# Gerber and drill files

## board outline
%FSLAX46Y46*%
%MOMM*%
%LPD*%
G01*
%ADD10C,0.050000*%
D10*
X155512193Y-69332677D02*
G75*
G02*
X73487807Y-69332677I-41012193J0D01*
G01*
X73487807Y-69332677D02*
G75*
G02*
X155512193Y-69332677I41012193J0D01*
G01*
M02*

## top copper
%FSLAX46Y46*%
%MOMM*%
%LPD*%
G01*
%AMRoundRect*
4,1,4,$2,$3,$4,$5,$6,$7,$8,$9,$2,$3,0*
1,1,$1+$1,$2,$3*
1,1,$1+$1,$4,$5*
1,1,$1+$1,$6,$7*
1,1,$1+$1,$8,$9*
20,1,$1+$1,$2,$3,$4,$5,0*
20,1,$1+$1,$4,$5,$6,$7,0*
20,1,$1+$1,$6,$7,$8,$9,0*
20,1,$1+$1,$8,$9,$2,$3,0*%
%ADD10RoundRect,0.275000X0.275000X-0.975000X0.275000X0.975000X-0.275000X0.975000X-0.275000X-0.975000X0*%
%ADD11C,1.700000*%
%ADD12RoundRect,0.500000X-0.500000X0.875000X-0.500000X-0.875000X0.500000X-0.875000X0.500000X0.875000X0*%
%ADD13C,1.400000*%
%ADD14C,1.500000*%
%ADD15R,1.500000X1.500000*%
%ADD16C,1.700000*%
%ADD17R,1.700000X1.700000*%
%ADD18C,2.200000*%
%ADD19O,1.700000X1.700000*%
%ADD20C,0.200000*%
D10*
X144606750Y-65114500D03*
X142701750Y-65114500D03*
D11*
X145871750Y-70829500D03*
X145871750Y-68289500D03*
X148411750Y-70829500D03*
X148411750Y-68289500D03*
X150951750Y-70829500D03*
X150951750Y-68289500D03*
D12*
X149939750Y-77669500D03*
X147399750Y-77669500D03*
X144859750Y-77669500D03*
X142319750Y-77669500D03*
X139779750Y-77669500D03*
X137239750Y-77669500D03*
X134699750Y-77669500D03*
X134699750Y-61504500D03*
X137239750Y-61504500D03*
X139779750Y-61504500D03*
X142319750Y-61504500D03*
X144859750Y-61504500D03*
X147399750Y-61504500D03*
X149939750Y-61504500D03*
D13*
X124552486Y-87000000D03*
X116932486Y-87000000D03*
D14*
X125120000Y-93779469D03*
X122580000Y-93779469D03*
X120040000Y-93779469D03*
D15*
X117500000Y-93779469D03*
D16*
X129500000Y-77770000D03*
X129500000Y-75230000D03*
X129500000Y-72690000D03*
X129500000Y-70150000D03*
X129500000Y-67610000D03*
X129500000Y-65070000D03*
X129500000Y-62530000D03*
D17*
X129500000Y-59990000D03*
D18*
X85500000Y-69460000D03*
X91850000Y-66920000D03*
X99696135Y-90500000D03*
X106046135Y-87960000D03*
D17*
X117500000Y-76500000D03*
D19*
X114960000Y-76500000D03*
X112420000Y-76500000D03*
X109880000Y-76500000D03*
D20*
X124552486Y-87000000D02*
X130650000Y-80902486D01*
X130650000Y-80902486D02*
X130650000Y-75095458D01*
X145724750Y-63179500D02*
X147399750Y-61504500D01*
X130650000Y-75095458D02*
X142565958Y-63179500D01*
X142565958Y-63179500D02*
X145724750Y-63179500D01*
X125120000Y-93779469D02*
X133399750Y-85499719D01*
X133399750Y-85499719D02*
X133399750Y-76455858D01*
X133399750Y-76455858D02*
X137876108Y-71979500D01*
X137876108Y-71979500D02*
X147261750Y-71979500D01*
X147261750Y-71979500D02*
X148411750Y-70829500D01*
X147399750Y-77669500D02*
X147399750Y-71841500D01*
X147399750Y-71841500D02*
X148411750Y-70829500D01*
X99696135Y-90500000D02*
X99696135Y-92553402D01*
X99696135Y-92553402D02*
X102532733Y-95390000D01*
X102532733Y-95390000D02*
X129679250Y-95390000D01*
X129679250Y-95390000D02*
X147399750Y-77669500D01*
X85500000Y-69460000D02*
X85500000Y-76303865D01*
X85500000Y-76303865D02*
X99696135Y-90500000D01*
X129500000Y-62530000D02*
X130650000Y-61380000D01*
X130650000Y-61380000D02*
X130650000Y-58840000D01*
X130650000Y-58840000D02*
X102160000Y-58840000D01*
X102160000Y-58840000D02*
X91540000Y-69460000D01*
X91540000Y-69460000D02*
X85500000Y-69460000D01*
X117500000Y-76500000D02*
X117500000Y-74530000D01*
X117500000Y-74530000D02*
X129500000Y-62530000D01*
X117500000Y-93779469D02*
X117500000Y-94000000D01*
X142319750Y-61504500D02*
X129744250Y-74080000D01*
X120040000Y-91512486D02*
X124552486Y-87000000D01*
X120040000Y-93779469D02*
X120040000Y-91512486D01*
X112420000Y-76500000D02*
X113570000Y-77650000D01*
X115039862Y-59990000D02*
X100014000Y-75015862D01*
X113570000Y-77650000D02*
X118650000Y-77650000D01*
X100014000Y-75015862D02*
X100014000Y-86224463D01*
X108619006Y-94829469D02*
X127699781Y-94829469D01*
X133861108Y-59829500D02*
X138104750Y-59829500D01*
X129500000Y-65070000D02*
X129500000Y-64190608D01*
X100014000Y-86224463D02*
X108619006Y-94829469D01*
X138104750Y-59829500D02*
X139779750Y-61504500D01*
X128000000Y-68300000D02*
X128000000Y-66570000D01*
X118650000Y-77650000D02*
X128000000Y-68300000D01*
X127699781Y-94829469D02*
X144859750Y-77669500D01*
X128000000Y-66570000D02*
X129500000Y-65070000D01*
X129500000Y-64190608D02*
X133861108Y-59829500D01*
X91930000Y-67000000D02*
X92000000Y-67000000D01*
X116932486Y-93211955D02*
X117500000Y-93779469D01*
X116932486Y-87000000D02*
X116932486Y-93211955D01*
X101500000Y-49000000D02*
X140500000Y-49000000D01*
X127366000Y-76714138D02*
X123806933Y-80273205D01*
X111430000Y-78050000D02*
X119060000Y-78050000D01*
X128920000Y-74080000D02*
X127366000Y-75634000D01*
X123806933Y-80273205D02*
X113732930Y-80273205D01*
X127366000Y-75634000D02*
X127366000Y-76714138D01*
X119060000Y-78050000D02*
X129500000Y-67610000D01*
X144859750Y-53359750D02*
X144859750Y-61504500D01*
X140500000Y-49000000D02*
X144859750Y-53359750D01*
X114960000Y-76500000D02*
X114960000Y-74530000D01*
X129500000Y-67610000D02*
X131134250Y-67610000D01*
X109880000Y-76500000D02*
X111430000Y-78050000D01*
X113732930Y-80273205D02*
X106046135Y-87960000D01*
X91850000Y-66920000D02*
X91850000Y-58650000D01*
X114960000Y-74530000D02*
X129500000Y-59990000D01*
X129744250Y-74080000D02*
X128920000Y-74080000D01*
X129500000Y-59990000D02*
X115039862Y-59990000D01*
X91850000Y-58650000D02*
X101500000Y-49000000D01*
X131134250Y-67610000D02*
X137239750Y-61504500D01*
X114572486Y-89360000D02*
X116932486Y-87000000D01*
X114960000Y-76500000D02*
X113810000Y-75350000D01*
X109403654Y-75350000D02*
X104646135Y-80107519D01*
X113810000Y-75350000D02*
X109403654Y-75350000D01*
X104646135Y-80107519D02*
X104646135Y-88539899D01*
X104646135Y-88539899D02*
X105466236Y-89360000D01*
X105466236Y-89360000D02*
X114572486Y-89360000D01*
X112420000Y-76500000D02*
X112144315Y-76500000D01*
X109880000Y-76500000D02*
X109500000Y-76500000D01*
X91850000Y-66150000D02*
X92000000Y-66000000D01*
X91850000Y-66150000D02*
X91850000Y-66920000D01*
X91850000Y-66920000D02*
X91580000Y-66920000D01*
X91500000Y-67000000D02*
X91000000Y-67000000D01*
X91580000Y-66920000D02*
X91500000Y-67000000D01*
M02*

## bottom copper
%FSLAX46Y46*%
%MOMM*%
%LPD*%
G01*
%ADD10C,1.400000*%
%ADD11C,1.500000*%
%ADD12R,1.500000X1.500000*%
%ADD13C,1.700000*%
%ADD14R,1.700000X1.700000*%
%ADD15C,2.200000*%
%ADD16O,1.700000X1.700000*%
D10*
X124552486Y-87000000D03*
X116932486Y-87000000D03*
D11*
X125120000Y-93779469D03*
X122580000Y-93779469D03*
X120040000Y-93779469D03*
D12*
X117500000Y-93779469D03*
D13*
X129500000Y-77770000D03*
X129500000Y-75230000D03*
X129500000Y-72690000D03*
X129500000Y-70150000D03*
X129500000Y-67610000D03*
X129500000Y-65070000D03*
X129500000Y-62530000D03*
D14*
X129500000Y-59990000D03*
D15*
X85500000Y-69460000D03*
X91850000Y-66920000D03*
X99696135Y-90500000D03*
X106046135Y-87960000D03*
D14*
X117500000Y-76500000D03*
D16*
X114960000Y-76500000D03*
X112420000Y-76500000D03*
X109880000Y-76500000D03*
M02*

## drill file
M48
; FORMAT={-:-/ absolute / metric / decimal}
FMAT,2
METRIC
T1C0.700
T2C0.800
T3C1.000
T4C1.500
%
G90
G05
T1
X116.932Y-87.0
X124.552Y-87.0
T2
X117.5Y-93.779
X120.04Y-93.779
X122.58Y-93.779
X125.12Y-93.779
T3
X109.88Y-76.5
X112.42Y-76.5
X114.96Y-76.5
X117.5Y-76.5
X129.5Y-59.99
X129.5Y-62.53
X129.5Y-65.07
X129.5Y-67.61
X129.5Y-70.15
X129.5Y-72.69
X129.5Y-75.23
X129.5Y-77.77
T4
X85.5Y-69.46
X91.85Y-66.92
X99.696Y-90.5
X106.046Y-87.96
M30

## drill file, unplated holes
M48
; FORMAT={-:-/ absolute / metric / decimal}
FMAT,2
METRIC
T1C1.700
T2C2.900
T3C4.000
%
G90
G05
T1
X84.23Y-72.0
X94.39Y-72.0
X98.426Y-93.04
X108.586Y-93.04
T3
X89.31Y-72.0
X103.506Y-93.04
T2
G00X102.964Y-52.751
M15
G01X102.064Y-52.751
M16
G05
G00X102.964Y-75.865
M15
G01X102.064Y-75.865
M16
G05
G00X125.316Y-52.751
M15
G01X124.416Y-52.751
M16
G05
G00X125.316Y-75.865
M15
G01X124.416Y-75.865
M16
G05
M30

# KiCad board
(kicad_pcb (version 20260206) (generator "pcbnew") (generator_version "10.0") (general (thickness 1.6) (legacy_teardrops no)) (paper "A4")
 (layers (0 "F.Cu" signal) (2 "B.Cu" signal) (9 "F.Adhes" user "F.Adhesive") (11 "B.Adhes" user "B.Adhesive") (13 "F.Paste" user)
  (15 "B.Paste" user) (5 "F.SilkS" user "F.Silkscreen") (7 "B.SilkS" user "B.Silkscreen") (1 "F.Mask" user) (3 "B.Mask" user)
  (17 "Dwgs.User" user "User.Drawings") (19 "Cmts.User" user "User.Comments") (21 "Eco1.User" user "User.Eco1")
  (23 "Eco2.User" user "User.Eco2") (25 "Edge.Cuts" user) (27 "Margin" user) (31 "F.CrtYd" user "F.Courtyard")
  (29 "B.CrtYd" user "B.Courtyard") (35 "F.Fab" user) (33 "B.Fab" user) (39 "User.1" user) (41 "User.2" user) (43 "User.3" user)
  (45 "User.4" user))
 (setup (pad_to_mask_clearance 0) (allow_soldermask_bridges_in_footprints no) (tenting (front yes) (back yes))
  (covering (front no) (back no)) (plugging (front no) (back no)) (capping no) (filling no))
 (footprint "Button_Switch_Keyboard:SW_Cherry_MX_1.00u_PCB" (layer "F.Cu") (at 106.046135 87.96)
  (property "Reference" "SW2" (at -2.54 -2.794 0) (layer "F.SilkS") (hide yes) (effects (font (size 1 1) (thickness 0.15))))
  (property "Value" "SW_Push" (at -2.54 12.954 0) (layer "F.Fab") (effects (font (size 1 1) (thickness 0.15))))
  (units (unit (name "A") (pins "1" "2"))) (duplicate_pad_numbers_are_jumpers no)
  (pad "" np_thru_hole circle (at -7.62 5.08) (size 1.7 1.7) (drill 1.7) (layers "*.Cu" "*.Mask"))
  (pad "" np_thru_hole circle (at -2.54 5.08) (size 4 4) (drill 4) (layers "*.Cu" "*.Mask"))
  (pad "" np_thru_hole circle (at 2.54 5.08) (size 1.7 1.7) (drill 1.7) (layers "*.Cu" "*.Mask"))
  (pad "1" thru_hole circle (at 0 0) (size 2.2 2.2) (drill 1.5) (layers "*.Cu" "*.Mask") (remove_unused_layers no) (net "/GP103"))
  (pad "2" thru_hole circle (at -6.35 2.54) (size 2.2 2.2) (drill 1.5) (layers "*.Cu" "*.Mask") (remove_unused_layers no) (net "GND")))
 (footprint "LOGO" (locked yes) (layer "F.Cu") (at 114.5 69.332677)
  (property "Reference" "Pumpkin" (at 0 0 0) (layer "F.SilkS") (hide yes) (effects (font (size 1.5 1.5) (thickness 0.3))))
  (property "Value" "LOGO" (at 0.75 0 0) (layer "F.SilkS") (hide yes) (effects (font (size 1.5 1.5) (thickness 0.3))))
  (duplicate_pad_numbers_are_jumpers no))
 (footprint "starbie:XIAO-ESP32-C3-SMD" (layer "F.Cu") (at 131.81975 60.6695 -90)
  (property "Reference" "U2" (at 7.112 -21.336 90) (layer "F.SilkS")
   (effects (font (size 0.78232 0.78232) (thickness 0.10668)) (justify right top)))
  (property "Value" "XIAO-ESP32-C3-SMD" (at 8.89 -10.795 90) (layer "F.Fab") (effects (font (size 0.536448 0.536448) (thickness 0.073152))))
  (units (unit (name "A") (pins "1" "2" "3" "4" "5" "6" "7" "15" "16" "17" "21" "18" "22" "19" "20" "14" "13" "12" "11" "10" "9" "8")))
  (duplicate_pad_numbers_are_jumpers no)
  (pad "1" smd roundrect (at 0.835 -18.12 270) (size 2.75 2) (layers "F.Cu" "F.Mask" "F.Paste") (roundrect_rratio 0.25)
   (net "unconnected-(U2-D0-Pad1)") (solder_mask_margin 0.0508) (thermal_bridge_angle 45))
  (pad "2" smd roundrect (at 0.835 -15.58 270) (size 2.75 2) (layers "F.Cu" "F.Mask" "F.Paste") (roundrect_rratio 0.25) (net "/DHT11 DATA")
   (solder_mask_margin 0.0508) (thermal_bridge_angle 45))
  (pad "3" smd roundrect (at 0.835 -13.04 270) (size 2.75 2) (layers "F.Cu" "F.Mask" "F.Paste") (roundrect_rratio 0.25) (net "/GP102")
   (solder_mask_margin 0.0508) (thermal_bridge_angle 45))
  (pad "4" smd roundrect (at 0.835 -10.5 270) (size 2.75 2) (layers "F.Cu" "F.Mask" "F.Paste") (roundrect_rratio 0.25) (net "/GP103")
   (solder_mask_margin 0.0508) (thermal_bridge_angle 45))
  (pad "5" smd roundrect (at 0.835 -7.96 270) (size 2.75 2) (layers "F.Cu" "F.Mask" "F.Paste") (roundrect_rratio 0.25) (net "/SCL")
   (solder_mask_margin 0.0508) (thermal_bridge_angle 45))
  (pad "6" smd roundrect (at 0.835 -5.42 270) (size 2.75 2) (layers "F.Cu" "F.Mask" "F.Paste") (roundrect_rratio 0.25) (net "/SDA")
   (solder_mask_margin 0.0508) (thermal_bridge_angle 45))
  (pad "7" smd roundrect (at 0.835 -2.88 270) (size 2.75 2) (layers "F.Cu" "F.Mask" "F.Paste") (roundrect_rratio 0.25)
   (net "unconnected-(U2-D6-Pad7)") (solder_mask_margin 0.0508) (thermal_bridge_angle 45))
  (pad "8" smd roundrect (at 17 -2.88 270) (size 2.75 2) (layers "F.Cu" "F.Mask" "F.Paste") (roundrect_rratio 0.25)
   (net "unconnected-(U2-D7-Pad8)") (solder_mask_margin 0.0508) (thermal_bridge_angle 45))
  (pad "9" smd roundrect (at 17 -5.42 270) (size 2.75 2) (layers "F.Cu" "F.Mask" "F.Paste") (roundrect_rratio 0.25)
   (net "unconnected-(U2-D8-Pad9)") (solder_mask_margin 0.0508) (thermal_bridge_angle 45))
  (pad "10" smd roundrect (at 17 -7.96 270) (size 2.75 2) (layers "F.Cu" "F.Mask" "F.Paste") (roundrect_rratio 0.25)
   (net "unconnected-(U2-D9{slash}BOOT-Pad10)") (solder_mask_margin 0.0508) (thermal_bridge_angle 45))
  (pad "11" smd roundrect (at 17 -10.5 270) (size 2.75 2) (layers "F.Cu" "F.Mask" "F.Paste") (roundrect_rratio 0.25)
   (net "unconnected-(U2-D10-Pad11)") (solder_mask_margin 0.0508) (thermal_bridge_angle 45))
  (pad "12" smd roundrect (at 17 -13.04 270) (size 2.75 2) (layers "F.Cu" "F.Mask" "F.Paste") (roundrect_rratio 0.25) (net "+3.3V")
   (solder_mask_margin 0.0508) (thermal_bridge_angle 45))
  (pad "13" smd roundrect (at 17 -15.58 270) (size 2.75 2) (layers "F.Cu" "F.Mask" "F.Paste") (roundrect_rratio 0.25) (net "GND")
   (solder_mask_margin 0.0508) (thermal_bridge_angle 45))
  (pad "14" smd roundrect (at 17 -18.12 270) (size 2.75 2) (layers "F.Cu" "F.Mask" "F.Paste") (roundrect_rratio 0.25) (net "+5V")
   (solder_mask_margin 0.0508) (thermal_bridge_angle 45))
  (pad "15" smd circle (at 7.62 -19.132 270) (size 1.7 1.7) (layers "F.Cu" "F.Mask" "F.Paste") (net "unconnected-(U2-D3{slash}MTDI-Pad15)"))
  (pad "16" smd circle (at 10.16 -19.132 270) (size 1.7 1.7) (layers "F.Cu" "F.Mask" "F.Paste") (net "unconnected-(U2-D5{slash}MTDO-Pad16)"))
  (pad "17" smd circle (at 7.62 -16.592 270) (size 1.7 1.7) (layers "F.Cu" "F.Mask" "F.Paste") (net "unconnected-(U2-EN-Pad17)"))
  (pad "18" smd circle (at 10.16 -16.592 270) (size 1.7 1.7) (layers "F.Cu" "F.Mask" "F.Paste") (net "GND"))
  (pad "19" smd circle (at 7.62 -14.052 270) (size 1.7 1.7) (layers "F.Cu" "F.Mask" "F.Paste") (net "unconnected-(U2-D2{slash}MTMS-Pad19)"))
  (pad "20" smd circle (at 10.16 -14.052 270) (size 1.7 1.7) (layers "F.Cu" "F.Mask" "F.Paste") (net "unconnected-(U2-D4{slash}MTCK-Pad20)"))
  (pad "21" smd roundrect (at 4.445 -10.882 90) (size 2.5 1.1) (layers "F.Cu" "F.Mask" "F.Paste") (roundrect_rratio 0.25)
   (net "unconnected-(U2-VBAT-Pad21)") (thermal_bridge_angle 45))
  (pad "22" smd roundrect (at 4.445 -12.787 90) (size 2.5 1.1) (layers "F.Cu" "F.Mask" "F.Paste") (roundrect_rratio 0.25)
   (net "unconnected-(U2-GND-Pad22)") (thermal_bridge_angle 45)))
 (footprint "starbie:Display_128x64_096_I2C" (layer "F.Cu") (at 113.69 76.5 180)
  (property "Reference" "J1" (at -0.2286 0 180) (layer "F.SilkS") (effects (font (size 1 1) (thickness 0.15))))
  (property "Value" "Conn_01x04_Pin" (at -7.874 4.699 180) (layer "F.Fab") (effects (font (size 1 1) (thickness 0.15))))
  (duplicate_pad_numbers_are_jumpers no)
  (pad "" np_thru_hole oval (at -11.176 0.635 180) (size 3.8 2.9) (drill oval 3.8 2.9) (layers "*.Cu" "*.Mask"))
  (pad "" np_thru_hole oval (at -11.176 23.749 180) (size 3.8 2.9) (drill oval 3.8 2.9) (layers "*.Cu" "*.Mask"))
  (pad "" np_thru_hole oval (at 11.176 0.635 180) (size 3.8 2.9) (drill oval 3.8 2.9) (layers "*.Cu" "*.Mask"))
  (pad "" np_thru_hole oval (at 11.176 23.749 180) (size 3.8 2.9) (drill oval 3.8 2.9) (layers "*.Cu" "*.Mask"))
  (pad "1" thru_hole rect (at -3.81 0 270) (size 1.7 1.7) (drill 1) (layers "*.Cu" "*.Mask") (remove_unused_layers no) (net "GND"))
  (pad "2" thru_hole oval (at -1.27 0 270) (size 1.7 1.7) (drill 1) (layers "*.Cu" "*.Mask") (remove_unused_layers no) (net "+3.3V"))
  (pad "3" thru_hole oval (at 1.27 0 270) (size 1.7 1.7) (drill 1) (layers "*.Cu" "*.Mask") (remove_unused_layers no) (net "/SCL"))
  (pad "4" thru_hole oval (at 3.81 0 270) (size 1.7 1.7) (drill 1) (layers "*.Cu" "*.Mask") (remove_unused_layers no) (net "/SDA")))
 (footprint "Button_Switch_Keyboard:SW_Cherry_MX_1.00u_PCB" (layer "F.Cu") (at 91.85 66.92)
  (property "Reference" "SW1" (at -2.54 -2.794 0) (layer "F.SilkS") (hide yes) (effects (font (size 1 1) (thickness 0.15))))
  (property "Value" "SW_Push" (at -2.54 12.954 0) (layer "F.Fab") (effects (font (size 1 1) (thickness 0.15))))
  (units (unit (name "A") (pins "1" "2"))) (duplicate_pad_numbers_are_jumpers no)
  (pad "" np_thru_hole circle (at -7.62 5.08) (size 1.7 1.7) (drill 1.7) (layers "*.Cu" "*.Mask"))
  (pad "" np_thru_hole circle (at -2.54 5.08) (size 4 4) (drill 4) (layers "*.Cu" "*.Mask"))
  (pad "" np_thru_hole circle (at 2.54 5.08) (size 1.7 1.7) (drill 1.7) (layers "*.Cu" "*.Mask"))
  (pad "1" thru_hole circle (at 0 0) (size 2.2 2.2) (drill 1.5) (layers "*.Cu" "*.Mask") (remove_unused_layers no) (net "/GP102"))
  (pad "2" thru_hole circle (at -6.35 2.54) (size 2.2 2.2) (drill 1.5) (layers "*.Cu" "*.Mask") (remove_unused_layers no) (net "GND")))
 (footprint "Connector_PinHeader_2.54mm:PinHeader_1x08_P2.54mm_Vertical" (layer "F.Cu") (at 129.5 59.99)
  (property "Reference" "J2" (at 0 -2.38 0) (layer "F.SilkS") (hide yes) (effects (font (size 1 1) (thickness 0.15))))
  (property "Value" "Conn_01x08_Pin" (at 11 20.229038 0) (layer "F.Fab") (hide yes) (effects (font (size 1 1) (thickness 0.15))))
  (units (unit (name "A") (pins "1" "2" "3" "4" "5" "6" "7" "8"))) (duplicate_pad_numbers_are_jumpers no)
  (pad "1" thru_hole rect (at 0 0) (size 1.7 1.7) (drill 1) (layers "*.Cu" "*.Mask") (remove_unused_layers no) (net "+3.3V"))
  (pad "2" thru_hole circle (at 0 2.54) (size 1.7 1.7) (drill 1) (layers "*.Cu" "*.Mask") (remove_unused_layers no) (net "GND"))
  (pad "3" thru_hole circle (at 0 5.08) (size 1.7 1.7) (drill 1) (layers "*.Cu" "*.Mask") (remove_unused_layers no) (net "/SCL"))
  (pad "4" thru_hole circle (at 0 7.62) (size 1.7 1.7) (drill 1) (layers "*.Cu" "*.Mask") (remove_unused_layers no) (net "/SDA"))
  (pad "5" thru_hole circle (at 0 10.16) (size 1.7 1.7) (drill 1) (layers "*.Cu" "*.Mask") (remove_unused_layers no)
   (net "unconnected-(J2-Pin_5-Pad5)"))
  (pad "6" thru_hole circle (at 0 12.7) (size 1.7 1.7) (drill 1) (layers "*.Cu" "*.Mask") (remove_unused_layers no)
   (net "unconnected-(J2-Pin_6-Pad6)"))
  (pad "7" thru_hole circle (at 0 15.24) (size 1.7 1.7) (drill 1) (layers "*.Cu" "*.Mask") (remove_unused_layers no)
   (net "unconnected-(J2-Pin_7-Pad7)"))
  (pad "8" thru_hole circle (at 0 17.78) (size 1.7 1.7) (drill 1) (layers "*.Cu" "*.Mask") (remove_unused_layers no)
   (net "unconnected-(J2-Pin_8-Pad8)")))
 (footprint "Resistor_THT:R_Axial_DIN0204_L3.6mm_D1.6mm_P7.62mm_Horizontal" (layer "F.Cu") (at 116.932486 87)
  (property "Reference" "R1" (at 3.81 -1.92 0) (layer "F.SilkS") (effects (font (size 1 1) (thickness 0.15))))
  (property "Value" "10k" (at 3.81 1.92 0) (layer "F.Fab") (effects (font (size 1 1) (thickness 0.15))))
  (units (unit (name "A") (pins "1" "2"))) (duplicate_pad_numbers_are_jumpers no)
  (pad "1" thru_hole circle (at 0 0) (size 1.4 1.4) (drill 0.7) (layers "*.Cu" "*.Mask") (remove_unused_layers no) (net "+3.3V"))
  (pad "2" thru_hole circle (at 7.62 0) (size 1.4 1.4) (drill 0.7) (layers "*.Cu" "*.Mask") (remove_unused_layers no) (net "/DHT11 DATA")))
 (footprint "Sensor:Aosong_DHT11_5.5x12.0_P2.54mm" (layer "F.Cu") (at 117.5 93.779469 90)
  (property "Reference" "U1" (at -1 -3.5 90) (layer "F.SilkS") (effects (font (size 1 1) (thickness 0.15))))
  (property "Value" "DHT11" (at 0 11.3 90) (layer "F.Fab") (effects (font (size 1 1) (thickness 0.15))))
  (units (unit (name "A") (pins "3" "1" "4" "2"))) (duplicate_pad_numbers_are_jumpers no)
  (pad "1" thru_hole rect (at 0 0 90) (size 1.5 1.5) (drill 0.8) (layers "*.Cu" "*.Mask") (remove_unused_layers no) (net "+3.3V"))
  (pad "2" thru_hole circle (at 0 2.54 90) (size 1.5 1.5) (drill 0.8) (layers "*.Cu" "*.Mask") (remove_unused_layers no) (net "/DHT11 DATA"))
  (pad "3" thru_hole circle (at 0 5.08 90) (size 1.5 1.5) (drill 0.8) (layers "*.Cu" "*.Mask") (remove_unused_layers no)
   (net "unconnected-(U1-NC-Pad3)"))
  (pad "4" thru_hole circle (at 0 7.62 90) (size 1.5 1.5) (drill 0.8) (layers "*.Cu" "*.Mask") (remove_unused_layers no) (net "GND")))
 (gr_circle (center 114.5 69.332677) (end 85.5 40.332677) (stroke (width 0.05) (type solid)) (fill no) (layer "Edge.Cuts"))
 (segment (start 113.73293 80.273205) (end 106.046135 87.96) (width 0.2) (layer "F.Cu") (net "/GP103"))
 (segment (start 128.92 74.08) (end 127.366 75.634) (width 0.2) (layer "F.Cu") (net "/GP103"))
 (segment (start 123.806933 80.273205) (end 113.73293 80.273205) (width 0.2) (layer "F.Cu") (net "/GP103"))
 (segment (start 127.366 76.714138) (end 123.806933 80.273205) (width 0.2) (layer "F.Cu") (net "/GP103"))
 (segment (start 142.31975 61.5045) (end 129.74425 74.08) (width 0.2) (layer "F.Cu") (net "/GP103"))
 (segment (start 129.74425 74.08) (end 128.92 74.08) (width 0.2) (layer "F.Cu") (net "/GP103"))
 (segment (start 127.366 75.634) (end 127.366 76.714138) (width 0.2) (layer "F.Cu") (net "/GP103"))
 (segment (start 133.39975 76.455858) (end 137.876108 71.9795) (width 0.2) (layer "F.Cu") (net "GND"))
 (segment (start 99.696135 92.553402) (end 102.532733 95.39) (width 0.2) (layer "F.Cu") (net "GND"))
 (segment (start 129.67925 95.39) (end 147.39975 77.6695) (width 0.2) (layer "F.Cu") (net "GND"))
 (segment (start 130.65 58.84) (end 102.16 58.84) (width 0.2) (layer "F.Cu") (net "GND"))
 (segment (start 91.54 69.46) (end 85.5 69.46) (width 0.2) (layer "F.Cu") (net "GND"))
 (segment (start 117.5 76.5) (end 117.5 74.53) (width 0.2) (layer "F.Cu") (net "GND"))
 (segment (start 102.16 58.84) (end 91.54 69.46) (width 0.2) (layer "F.Cu") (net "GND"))
 (segment (start 129.5 62.53) (end 130.65 61.38) (width 0.2) (layer "F.Cu") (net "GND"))
 (segment (start 102.532733 95.39) (end 129.67925 95.39) (width 0.2) (layer "F.Cu") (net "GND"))
 (segment (start 147.39975 71.8415) (end 148.41175 70.8295) (width 0.2) (layer "F.Cu") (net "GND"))
 (segment (start 125.12 93.779469) (end 133.39975 85.499719) (width 0.2) (layer "F.Cu") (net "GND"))
 (segment (start 130.65 61.38) (end 130.65 58.84) (width 0.2) (layer "F.Cu") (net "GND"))
 (segment (start 133.39975 85.499719) (end 133.39975 76.455858) (width 0.2) (layer "F.Cu") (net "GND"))
 (segment (start 85.5 76.303865) (end 99.696135 90.5) (width 0.2) (layer "F.Cu") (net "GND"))
 (segment (start 147.39975 77.6695) (end 147.39975 71.8415) (width 0.2) (layer "F.Cu") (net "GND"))
 (segment (start 147.26175 71.9795) (end 148.41175 70.8295) (width 0.2) (layer "F.Cu") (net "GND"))
 (segment (start 85.5 69.46) (end 85.5 76.303865) (width 0.2) (layer "F.Cu") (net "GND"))
 (segment (start 137.876108 71.9795) (end 147.26175 71.9795) (width 0.2) (layer "F.Cu") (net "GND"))
 (segment (start 99.696135 90.5) (end 99.696135 92.553402) (width 0.2) (layer "F.Cu") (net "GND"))
 (segment (start 117.5 74.53) (end 129.5 62.53) (width 0.2) (layer "F.Cu") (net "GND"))
 (segment (start 130.65 80.902486) (end 130.65 75.095458) (width 0.2) (layer "F.Cu") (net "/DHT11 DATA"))
 (segment (start 120.04 93.779469) (end 120.04 91.512486) (width 0.2) (layer "F.Cu") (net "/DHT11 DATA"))
 (segment (start 120.04 91.512486) (end 124.552486 87) (width 0.2) (layer "F.Cu") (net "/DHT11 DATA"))
 (segment (start 130.65 75.095458) (end 142.565958 63.1795) (width 0.2) (layer "F.Cu") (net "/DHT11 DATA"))
 (segment (start 124.552486 87) (end 130.65 80.902486) (width 0.2) (layer "F.Cu") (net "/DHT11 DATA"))
 (segment (start 145.72475 63.1795) (end 147.39975 61.5045) (width 0.2) (layer "F.Cu") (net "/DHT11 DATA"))
 (segment (start 142.565958 63.1795) (end 145.72475 63.1795) (width 0.2) (layer "F.Cu") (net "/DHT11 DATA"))
 (segment (start 91.85 66.92) (end 91.85 58.65) (width 0.2) (layer "F.Cu") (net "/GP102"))
 (segment (start 91.58 66.92) (end 91.5 67) (width 0.2) (layer "F.Cu") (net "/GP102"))
 (segment (start 91.85 66.92) (end 91.58 66.92) (width 0.2) (layer "F.Cu") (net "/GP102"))
 (segment (start 101.5 49) (end 140.5 49) (width 0.2) (layer "F.Cu") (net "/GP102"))
 (segment (start 91.85 58.65) (end 101.5 49) (width 0.2) (layer "F.Cu") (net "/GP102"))
 (segment (start 91.5 67) (end 91 67) (width 0.2) (layer "F.Cu") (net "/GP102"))
 (segment (start 144.85975 53.35975) (end 144.85975 61.5045) (width 0.2) (layer "F.Cu") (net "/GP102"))
 (segment (start 140.5 49) (end 144.85975 53.35975) (width 0.2) (layer "F.Cu") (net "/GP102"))
 (segment (start 91.85 66.15) (end 91.85 66.92) (width 0.2) (layer "F.Cu") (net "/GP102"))
 (segment (start 91.93 67) (end 92 67) (width 0.2) (layer "F.Cu") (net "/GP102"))
 (segment (start 91.85 66.15) (end 92 66) (width 0.2) (layer "F.Cu") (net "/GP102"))
 (segment (start 109.88 76.5) (end 109.5 76.5) (width 0.2) (layer "F.Cu") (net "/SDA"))
 (segment (start 111.43 78.05) (end 119.06 78.05) (width 0.2) (layer "F.Cu") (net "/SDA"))
 (segment (start 129.5 67.61) (end 131.13425 67.61) (width 0.2) (layer "F.Cu") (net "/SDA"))
 (segment (start 131.13425 67.61) (end 137.23975 61.5045) (width 0.2) (layer "F.Cu") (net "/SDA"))
 (segment (start 119.06 78.05) (end 129.5 67.61) (width 0.2) (layer "F.Cu") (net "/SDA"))
 (segment (start 109.88 76.5) (end 111.43 78.05) (width 0.2) (layer "F.Cu") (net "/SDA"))
 (segment (start 116.932486 87) (end 116.932486 93.211955) (width 0.2) (layer "F.Cu") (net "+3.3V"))
 (segment (start 114.96 76.5) (end 114.96 74.53) (width 0.2) (layer "F.Cu") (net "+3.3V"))
 (segment (start 104.646135 80.107519) (end 104.646135 88.539899) (width 0.2) (layer "F.Cu") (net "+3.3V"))
 (segment (start 129.5 59.99) (end 115.039862 59.99) (width 0.2) (layer "F.Cu") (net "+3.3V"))
 (segment (start 108.619006 94.829469) (end 127.699781 94.829469) (width 0.2) (layer "F.Cu") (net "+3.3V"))
 (segment (start 117.5 93.779469) (end 117.5 94) (width 0.2) (layer "F.Cu") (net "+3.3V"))
 (segment (start 113.81 75.35) (end 109.403654 75.35) (width 0.2) (layer "F.Cu") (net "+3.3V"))
 (segment (start 127.699781 94.829469) (end 144.85975 77.6695) (width 0.2) (layer "F.Cu") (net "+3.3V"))
 (segment (start 115.039862 59.99) (end 100.014 75.015862) (width 0.2) (layer "F.Cu") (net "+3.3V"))
 (segment (start 100.014 75.015862) (end 100.014 86.224463) (width 0.2) (layer "F.Cu") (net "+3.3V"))
 (segment (start 105.466236 89.36) (end 114.572486 89.36) (width 0.2) (layer "F.Cu") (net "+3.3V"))
 (segment (start 114.96 76.5) (end 113.81 75.35) (width 0.2) (layer "F.Cu") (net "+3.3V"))
 (segment (start 114.572486 89.36) (end 116.932486 87) (width 0.2) (layer "F.Cu") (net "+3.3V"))
 (segment (start 104.646135 88.539899) (end 105.466236 89.36) (width 0.2) (layer "F.Cu") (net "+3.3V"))
 (segment (start 114.96 74.53) (end 129.5 59.99) (width 0.2) (layer "F.Cu") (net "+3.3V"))
 (segment (start 109.403654 75.35) (end 104.646135 80.107519) (width 0.2) (layer "F.Cu") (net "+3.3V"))
 (segment (start 100.014 86.224463) (end 108.619006 94.829469) (width 0.2) (layer "F.Cu") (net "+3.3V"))
 (segment (start 116.932486 93.211955) (end 117.5 93.779469) (width 0.2) (layer "F.Cu") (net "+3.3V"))
 (segment (start 112.42 76.5) (end 112.144315 76.5) (width 0.2) (layer "F.Cu") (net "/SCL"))
 (segment (start 118.65 77.65) (end 128 68.3) (width 0.2) (layer "F.Cu") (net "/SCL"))
 (segment (start 129.5 64.190608) (end 133.861108 59.8295) (width 0.2) (layer "F.Cu") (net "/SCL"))
 (segment (start 128 66.57) (end 129.5 65.07) (width 0.2) (layer "F.Cu") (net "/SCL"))
 (segment (start 133.861108 59.8295) (end 138.10475 59.8295) (width 0.2) (layer "F.Cu") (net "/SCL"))
 (segment (start 112.42 76.5) (end 113.57 77.65) (width 0.2) (layer "F.Cu") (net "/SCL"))
 (segment (start 138.10475 59.8295) (end 139.77975 61.5045) (width 0.2) (layer "F.Cu") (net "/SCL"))
 (segment (start 129.5 65.07) (end 129.5 64.190608) (width 0.2) (layer "F.Cu") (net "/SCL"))
 (segment (start 113.57 77.65) (end 118.65 77.65) (width 0.2) (layer "F.Cu") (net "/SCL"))
 (segment (start 128 68.3) (end 128 66.57) (width 0.2) (layer "F.Cu") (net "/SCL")))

